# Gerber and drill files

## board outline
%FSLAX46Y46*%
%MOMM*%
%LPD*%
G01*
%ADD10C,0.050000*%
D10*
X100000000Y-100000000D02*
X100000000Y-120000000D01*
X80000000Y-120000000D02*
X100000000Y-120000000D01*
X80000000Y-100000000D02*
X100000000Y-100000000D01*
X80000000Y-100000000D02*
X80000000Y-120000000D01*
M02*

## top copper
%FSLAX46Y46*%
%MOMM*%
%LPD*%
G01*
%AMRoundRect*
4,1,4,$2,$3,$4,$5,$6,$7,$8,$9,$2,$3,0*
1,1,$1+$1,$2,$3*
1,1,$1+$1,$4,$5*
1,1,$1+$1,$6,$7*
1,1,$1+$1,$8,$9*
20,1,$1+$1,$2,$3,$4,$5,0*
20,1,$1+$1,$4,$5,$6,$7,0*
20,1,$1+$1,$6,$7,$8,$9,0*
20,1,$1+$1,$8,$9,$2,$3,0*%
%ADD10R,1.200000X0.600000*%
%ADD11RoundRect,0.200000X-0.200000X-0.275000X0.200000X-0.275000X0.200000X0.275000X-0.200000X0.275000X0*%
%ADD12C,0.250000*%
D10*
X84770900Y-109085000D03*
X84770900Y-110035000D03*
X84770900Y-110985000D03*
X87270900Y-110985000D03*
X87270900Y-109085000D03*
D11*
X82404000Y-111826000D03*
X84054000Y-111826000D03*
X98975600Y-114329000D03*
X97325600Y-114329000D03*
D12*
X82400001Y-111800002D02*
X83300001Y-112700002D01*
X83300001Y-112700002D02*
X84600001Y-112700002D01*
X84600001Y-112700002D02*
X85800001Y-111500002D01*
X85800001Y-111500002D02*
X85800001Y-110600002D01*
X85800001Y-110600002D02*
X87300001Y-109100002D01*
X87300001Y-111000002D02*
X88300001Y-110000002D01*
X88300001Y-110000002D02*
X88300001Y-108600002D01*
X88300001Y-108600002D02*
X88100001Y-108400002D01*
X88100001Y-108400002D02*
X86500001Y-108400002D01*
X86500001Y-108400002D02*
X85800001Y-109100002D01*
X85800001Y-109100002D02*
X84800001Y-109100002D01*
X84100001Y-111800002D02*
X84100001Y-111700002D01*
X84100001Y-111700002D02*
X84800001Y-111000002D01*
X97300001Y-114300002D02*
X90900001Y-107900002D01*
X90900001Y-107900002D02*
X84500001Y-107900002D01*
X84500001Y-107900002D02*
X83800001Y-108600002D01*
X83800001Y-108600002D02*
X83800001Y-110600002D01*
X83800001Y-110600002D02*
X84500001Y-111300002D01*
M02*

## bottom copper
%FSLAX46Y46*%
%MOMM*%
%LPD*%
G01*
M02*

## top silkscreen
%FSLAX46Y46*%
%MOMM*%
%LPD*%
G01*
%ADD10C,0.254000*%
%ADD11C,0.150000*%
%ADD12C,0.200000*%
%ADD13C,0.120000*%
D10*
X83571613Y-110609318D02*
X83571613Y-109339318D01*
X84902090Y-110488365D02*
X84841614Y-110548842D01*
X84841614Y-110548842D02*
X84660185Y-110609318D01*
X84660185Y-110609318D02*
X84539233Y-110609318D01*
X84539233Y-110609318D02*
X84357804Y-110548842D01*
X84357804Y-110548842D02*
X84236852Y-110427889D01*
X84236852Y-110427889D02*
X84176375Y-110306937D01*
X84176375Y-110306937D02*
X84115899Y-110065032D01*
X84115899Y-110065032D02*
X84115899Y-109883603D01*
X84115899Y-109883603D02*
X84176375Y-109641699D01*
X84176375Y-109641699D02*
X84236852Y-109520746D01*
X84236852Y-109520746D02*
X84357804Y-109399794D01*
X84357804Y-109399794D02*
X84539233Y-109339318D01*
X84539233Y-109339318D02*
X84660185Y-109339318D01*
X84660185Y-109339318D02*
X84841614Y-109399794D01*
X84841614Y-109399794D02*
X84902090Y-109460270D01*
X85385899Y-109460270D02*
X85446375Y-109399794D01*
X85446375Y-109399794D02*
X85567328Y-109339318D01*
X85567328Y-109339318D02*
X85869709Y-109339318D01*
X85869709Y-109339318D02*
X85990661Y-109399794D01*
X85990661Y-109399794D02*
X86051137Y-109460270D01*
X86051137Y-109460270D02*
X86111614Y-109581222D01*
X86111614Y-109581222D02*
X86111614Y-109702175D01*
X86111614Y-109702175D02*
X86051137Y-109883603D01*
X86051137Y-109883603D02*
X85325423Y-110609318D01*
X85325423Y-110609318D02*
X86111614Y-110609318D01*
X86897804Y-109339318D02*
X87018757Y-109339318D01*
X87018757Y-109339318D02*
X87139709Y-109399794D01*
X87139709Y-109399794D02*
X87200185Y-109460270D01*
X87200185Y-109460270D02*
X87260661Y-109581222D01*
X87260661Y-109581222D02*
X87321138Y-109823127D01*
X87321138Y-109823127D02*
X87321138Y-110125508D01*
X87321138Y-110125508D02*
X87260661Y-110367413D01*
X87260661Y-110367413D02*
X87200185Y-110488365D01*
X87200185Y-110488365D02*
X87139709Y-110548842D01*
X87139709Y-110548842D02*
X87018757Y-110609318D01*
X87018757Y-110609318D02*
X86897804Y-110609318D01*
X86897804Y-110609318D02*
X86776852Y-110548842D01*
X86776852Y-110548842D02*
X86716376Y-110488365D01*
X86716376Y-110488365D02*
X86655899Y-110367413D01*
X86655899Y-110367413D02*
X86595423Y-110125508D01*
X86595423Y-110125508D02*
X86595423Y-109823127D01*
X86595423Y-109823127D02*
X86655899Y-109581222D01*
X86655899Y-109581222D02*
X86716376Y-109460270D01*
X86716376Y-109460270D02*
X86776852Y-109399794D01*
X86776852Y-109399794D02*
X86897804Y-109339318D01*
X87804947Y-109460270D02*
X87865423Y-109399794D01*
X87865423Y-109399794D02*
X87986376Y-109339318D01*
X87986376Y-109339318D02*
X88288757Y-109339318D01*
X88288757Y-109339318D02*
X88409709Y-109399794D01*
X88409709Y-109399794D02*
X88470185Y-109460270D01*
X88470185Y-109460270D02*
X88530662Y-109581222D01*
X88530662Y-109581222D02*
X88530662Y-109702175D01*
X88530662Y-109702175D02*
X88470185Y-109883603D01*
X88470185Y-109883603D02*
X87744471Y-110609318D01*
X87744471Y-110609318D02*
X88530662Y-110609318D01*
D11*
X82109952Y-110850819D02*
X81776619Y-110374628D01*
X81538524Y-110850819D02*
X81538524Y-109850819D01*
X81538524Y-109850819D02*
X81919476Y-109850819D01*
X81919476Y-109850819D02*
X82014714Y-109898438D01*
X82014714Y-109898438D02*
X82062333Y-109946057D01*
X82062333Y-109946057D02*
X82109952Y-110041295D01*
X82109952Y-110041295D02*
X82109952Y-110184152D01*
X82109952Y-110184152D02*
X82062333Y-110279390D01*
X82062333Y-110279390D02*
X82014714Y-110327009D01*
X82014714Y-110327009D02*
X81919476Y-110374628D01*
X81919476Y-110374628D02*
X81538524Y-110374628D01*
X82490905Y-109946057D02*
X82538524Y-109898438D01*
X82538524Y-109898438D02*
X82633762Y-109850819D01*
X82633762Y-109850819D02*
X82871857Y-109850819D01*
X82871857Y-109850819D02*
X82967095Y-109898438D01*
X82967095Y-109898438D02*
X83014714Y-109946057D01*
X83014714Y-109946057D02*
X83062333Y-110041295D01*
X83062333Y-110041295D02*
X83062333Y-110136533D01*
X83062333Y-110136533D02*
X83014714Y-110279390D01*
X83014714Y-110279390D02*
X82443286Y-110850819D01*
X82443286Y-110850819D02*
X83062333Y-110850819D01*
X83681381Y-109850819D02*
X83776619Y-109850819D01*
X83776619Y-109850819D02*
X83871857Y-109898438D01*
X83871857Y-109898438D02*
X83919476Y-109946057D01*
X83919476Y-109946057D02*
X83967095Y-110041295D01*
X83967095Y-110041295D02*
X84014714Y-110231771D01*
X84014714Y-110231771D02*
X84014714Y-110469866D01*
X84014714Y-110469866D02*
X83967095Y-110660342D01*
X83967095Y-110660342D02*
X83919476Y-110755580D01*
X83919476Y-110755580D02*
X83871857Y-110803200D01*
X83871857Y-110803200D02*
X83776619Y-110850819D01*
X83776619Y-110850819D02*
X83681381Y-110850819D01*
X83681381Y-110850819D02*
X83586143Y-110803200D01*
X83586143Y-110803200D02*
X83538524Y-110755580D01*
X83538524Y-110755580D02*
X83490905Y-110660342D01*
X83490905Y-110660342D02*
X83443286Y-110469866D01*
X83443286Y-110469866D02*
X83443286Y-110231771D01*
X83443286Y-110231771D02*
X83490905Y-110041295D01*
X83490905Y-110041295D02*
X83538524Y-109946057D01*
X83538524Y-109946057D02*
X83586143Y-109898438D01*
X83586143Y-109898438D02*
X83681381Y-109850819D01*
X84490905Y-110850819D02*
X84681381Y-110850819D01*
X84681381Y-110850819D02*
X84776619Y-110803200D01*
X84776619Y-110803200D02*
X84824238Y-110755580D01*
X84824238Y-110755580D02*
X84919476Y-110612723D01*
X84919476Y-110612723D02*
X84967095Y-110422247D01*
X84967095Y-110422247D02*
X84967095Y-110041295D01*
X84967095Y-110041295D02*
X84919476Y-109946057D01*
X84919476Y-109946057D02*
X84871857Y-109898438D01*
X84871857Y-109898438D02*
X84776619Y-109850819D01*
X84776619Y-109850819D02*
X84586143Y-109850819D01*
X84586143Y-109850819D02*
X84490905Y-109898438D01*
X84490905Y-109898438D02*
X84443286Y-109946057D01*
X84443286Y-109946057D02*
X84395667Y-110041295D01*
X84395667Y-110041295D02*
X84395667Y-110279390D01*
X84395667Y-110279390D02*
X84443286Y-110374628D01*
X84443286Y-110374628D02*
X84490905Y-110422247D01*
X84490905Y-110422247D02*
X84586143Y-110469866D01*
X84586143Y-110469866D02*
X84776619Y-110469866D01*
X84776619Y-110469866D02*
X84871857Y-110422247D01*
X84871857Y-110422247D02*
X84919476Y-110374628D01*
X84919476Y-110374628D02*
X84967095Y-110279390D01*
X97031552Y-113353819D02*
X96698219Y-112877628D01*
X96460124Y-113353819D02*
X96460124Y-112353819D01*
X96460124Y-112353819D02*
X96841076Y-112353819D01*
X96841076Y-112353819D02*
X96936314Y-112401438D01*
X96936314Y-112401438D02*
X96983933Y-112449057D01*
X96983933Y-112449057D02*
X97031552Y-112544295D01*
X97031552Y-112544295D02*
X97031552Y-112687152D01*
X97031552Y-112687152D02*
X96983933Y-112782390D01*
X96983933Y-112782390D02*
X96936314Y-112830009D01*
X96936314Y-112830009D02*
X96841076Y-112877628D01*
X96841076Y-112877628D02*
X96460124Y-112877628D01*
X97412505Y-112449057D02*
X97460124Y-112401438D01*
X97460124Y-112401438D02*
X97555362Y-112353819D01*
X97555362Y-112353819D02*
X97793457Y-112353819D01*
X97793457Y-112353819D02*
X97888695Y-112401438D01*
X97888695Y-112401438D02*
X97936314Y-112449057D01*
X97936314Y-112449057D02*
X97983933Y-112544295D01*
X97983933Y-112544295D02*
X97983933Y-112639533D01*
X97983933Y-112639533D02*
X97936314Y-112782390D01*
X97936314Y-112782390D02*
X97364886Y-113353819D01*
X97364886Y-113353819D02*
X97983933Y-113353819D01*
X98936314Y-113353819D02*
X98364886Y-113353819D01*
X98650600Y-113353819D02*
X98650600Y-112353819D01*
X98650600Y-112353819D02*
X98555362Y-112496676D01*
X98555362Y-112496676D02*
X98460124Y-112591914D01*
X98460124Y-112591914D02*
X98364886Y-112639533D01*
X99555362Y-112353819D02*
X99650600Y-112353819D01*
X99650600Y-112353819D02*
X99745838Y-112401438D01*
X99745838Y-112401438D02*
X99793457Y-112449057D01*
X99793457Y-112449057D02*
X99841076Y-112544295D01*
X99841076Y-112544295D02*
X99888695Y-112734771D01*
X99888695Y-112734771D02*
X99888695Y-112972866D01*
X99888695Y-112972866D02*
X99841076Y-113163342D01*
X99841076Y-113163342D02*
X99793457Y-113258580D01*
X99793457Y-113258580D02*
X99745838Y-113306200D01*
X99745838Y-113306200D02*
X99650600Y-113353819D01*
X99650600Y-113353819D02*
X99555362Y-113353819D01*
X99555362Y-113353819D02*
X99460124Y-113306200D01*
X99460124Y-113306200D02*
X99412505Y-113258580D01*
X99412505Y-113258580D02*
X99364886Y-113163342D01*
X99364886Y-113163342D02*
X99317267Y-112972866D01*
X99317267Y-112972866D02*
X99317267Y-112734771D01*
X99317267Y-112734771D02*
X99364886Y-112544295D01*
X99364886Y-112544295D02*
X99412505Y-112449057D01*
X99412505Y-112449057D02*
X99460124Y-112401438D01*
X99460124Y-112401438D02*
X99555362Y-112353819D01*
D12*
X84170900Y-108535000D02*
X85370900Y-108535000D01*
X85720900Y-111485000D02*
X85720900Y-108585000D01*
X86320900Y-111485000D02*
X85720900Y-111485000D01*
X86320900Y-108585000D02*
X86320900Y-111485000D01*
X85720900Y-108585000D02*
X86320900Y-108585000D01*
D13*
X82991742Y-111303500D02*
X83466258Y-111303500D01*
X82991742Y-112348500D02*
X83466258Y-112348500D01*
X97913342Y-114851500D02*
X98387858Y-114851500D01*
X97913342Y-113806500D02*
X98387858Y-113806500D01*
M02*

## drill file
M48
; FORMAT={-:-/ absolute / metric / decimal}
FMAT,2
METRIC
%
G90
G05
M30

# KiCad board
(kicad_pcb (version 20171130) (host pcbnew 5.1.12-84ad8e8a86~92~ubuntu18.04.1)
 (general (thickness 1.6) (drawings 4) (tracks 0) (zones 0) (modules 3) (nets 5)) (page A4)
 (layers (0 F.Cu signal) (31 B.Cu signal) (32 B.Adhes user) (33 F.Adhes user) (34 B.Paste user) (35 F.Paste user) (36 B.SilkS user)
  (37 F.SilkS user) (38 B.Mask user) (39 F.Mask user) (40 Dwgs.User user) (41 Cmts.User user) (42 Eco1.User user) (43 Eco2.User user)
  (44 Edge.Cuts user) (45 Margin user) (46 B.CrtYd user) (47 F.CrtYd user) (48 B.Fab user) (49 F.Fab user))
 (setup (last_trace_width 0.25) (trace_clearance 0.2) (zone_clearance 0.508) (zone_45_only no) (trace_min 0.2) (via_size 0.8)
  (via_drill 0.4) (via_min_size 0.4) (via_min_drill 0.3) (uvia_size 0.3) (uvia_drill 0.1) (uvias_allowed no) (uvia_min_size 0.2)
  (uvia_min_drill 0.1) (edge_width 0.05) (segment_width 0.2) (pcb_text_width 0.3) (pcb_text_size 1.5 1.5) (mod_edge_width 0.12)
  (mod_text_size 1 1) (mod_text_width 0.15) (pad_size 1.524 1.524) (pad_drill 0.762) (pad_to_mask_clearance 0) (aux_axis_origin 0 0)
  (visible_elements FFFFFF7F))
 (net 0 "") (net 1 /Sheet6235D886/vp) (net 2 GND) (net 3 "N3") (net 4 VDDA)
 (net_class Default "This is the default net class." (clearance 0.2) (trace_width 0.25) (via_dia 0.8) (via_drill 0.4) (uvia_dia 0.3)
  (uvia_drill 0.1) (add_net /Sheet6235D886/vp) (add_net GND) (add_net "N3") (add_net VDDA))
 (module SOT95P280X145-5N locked (layer F.Cu) (at 86.020900 110.035000)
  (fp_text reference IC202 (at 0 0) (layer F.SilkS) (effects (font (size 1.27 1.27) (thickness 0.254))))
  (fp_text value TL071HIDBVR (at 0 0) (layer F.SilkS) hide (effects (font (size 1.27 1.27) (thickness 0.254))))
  (fp_line (start -1.85 -1.5) (end -0.65 -1.5) (layer F.SilkS) (width 0.2))
  (fp_line (start -0.3 1.45) (end -0.3 -1.45) (layer F.SilkS) (width 0.2))
  (fp_line (start 0.3 1.45) (end -0.3 1.45) (layer F.SilkS) (width 0.2))
  (fp_line (start 0.3 -1.45) (end 0.3 1.45) (layer F.SilkS) (width 0.2))
  (fp_line (start -0.3 -1.45) (end 0.3 -1.45) (layer F.SilkS) (width 0.2))
  (pad 1 smd rect (at -1.25 -0.95 90.000000) (size 0.6 1.2) (layers F.Cu F.Mask F.Paste) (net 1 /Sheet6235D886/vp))
  (pad 2 smd rect (at -1.25 0 90.000000) (size 0.6 1.2) (layers F.Cu F.Mask F.Paste) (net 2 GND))
  (pad 3 smd rect (at -1.25 0.95 90.000000) (size 0.6 1.2) (layers F.Cu F.Mask F.Paste) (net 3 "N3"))
  (pad 4 smd rect (at 1.25 0.95 90.000000) (size 0.6 1.2) (layers F.Cu F.Mask F.Paste) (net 1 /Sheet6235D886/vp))
  (pad 5 smd rect (at 1.25 -0.95 90.000000) (size 0.6 1.2) (layers F.Cu F.Mask F.Paste) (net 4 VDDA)))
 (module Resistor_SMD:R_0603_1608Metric (layer F.Cu) (at 83.229000 111.826000)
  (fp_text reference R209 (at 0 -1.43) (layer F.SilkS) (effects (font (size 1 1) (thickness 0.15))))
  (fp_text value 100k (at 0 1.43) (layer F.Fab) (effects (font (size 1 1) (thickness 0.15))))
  (fp_line (start -0.237258 -0.5225) (end 0.237258 -0.5225) (layer F.SilkS) (width 0.12))
  (fp_line (start -0.237258 0.5225) (end 0.237258 0.5225) (layer F.SilkS) (width 0.12))
  (pad 1 smd roundrect (at -0.825 0) (size 0.8 0.95) (layers F.Cu F.Mask F.Paste) (roundrect_rratio 0.25) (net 4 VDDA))
  (pad 2 smd roundrect (at 0.825 0) (size 0.8 0.95) (layers F.Cu F.Mask F.Paste) (roundrect_rratio 0.25) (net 3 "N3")))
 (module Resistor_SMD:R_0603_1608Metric (layer F.Cu) (at 98.150600 114.329000)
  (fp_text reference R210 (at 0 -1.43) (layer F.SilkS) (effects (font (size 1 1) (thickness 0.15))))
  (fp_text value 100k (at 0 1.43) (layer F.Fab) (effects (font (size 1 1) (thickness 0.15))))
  (fp_line (start -0.237258 0.5225) (end 0.237258 0.5225) (layer F.SilkS) (width 0.12))
  (fp_line (start -0.237258 -0.5225) (end 0.237258 -0.5225) (layer F.SilkS) (width 0.12))
  (pad 2 smd roundrect (at 0.825 0) (size 0.8 0.95) (layers F.Cu F.Mask F.Paste) (roundrect_rratio 0.25) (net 2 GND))
  (pad 1 smd roundrect (at -0.825 0) (size 0.8 0.95) (layers F.Cu F.Mask F.Paste) (roundrect_rratio 0.25) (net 3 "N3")))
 (gr_line (start 100 100) (end 100 120) (layer Edge.Cuts) (width 0.05))
 (gr_line (start 80 120) (end 100 120) (layer Edge.Cuts) (width 0.05))
 (gr_line (start 80 100) (end 100 100) (layer Edge.Cuts) (width 0.05))
 (gr_line (start 80 100) (end 80 120) (layer Edge.Cuts) (width 0.05))
 (segment (start 82.400001 111.800002) (end 83.300001 112.700002) (width 0.250000) (layer F.Cu) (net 4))
 (segment (start 83.300001 112.700002) (end 84.600001 112.700002) (width 0.250000) (layer F.Cu) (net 4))
 (segment (start 84.600001 112.700002) (end 85.800001 111.500002) (width 0.250000) (layer F.Cu) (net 4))
 (segment (start 85.800001 111.500002) (end 85.800001 110.600002) (width 0.250000) (layer F.Cu) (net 4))
 (segment (start 85.800001 110.600002) (end 87.300001 109.100002) (width 0.250000) (layer F.Cu) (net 4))
 (segment (start 87.300001 111.000002) (end 88.300001 110.000002) (width 0.250000) (layer F.Cu) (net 1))
 (segment (start 88.300001 110.000002) (end 88.300001 108.600002) (width 0.250000) (layer F.Cu) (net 1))
 (segment (start 88.300001 108.600002) (end 88.100001 108.400002) (width 0.250000) (layer F.Cu) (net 1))
 (segment (start 88.100001 108.400002) (end 86.500001 108.400002) (width 0.250000) (layer F.Cu) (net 1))
 (segment (start 86.500001 108.400002) (end 85.800001 109.100002) (width 0.250000) (layer F.Cu) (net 1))
 (segment (start 85.800001 109.100002) (end 84.800001 109.100002) (width 0.250000) (layer F.Cu) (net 1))
 (segment (start 84.100001 111.800002) (end 84.100001 111.700002) (width 0.250000) (layer F.Cu) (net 3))
 (segment (start 84.100001 111.700002) (end 84.800001 111.000002) (width 0.250000) (layer F.Cu) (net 3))
 (segment (start 97.300001 114.300002) (end 90.900001 107.900002) (width 0.250000) (layer F.Cu) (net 3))
 (segment (start 90.900001 107.900002) (end 84.500001 107.900002) (width 0.250000) (layer F.Cu) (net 3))
 (segment (start 84.500001 107.900002) (end 83.800001 108.600002) (width 0.250000) (layer F.Cu) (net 3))
 (segment (start 83.800001 108.600002) (end 83.800001 110.600002) (width 0.250000) (layer F.Cu) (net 3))
 (segment (start 83.800001 110.600002) (end 84.500001 111.300002) (width 0.250000) (layer F.Cu) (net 3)))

